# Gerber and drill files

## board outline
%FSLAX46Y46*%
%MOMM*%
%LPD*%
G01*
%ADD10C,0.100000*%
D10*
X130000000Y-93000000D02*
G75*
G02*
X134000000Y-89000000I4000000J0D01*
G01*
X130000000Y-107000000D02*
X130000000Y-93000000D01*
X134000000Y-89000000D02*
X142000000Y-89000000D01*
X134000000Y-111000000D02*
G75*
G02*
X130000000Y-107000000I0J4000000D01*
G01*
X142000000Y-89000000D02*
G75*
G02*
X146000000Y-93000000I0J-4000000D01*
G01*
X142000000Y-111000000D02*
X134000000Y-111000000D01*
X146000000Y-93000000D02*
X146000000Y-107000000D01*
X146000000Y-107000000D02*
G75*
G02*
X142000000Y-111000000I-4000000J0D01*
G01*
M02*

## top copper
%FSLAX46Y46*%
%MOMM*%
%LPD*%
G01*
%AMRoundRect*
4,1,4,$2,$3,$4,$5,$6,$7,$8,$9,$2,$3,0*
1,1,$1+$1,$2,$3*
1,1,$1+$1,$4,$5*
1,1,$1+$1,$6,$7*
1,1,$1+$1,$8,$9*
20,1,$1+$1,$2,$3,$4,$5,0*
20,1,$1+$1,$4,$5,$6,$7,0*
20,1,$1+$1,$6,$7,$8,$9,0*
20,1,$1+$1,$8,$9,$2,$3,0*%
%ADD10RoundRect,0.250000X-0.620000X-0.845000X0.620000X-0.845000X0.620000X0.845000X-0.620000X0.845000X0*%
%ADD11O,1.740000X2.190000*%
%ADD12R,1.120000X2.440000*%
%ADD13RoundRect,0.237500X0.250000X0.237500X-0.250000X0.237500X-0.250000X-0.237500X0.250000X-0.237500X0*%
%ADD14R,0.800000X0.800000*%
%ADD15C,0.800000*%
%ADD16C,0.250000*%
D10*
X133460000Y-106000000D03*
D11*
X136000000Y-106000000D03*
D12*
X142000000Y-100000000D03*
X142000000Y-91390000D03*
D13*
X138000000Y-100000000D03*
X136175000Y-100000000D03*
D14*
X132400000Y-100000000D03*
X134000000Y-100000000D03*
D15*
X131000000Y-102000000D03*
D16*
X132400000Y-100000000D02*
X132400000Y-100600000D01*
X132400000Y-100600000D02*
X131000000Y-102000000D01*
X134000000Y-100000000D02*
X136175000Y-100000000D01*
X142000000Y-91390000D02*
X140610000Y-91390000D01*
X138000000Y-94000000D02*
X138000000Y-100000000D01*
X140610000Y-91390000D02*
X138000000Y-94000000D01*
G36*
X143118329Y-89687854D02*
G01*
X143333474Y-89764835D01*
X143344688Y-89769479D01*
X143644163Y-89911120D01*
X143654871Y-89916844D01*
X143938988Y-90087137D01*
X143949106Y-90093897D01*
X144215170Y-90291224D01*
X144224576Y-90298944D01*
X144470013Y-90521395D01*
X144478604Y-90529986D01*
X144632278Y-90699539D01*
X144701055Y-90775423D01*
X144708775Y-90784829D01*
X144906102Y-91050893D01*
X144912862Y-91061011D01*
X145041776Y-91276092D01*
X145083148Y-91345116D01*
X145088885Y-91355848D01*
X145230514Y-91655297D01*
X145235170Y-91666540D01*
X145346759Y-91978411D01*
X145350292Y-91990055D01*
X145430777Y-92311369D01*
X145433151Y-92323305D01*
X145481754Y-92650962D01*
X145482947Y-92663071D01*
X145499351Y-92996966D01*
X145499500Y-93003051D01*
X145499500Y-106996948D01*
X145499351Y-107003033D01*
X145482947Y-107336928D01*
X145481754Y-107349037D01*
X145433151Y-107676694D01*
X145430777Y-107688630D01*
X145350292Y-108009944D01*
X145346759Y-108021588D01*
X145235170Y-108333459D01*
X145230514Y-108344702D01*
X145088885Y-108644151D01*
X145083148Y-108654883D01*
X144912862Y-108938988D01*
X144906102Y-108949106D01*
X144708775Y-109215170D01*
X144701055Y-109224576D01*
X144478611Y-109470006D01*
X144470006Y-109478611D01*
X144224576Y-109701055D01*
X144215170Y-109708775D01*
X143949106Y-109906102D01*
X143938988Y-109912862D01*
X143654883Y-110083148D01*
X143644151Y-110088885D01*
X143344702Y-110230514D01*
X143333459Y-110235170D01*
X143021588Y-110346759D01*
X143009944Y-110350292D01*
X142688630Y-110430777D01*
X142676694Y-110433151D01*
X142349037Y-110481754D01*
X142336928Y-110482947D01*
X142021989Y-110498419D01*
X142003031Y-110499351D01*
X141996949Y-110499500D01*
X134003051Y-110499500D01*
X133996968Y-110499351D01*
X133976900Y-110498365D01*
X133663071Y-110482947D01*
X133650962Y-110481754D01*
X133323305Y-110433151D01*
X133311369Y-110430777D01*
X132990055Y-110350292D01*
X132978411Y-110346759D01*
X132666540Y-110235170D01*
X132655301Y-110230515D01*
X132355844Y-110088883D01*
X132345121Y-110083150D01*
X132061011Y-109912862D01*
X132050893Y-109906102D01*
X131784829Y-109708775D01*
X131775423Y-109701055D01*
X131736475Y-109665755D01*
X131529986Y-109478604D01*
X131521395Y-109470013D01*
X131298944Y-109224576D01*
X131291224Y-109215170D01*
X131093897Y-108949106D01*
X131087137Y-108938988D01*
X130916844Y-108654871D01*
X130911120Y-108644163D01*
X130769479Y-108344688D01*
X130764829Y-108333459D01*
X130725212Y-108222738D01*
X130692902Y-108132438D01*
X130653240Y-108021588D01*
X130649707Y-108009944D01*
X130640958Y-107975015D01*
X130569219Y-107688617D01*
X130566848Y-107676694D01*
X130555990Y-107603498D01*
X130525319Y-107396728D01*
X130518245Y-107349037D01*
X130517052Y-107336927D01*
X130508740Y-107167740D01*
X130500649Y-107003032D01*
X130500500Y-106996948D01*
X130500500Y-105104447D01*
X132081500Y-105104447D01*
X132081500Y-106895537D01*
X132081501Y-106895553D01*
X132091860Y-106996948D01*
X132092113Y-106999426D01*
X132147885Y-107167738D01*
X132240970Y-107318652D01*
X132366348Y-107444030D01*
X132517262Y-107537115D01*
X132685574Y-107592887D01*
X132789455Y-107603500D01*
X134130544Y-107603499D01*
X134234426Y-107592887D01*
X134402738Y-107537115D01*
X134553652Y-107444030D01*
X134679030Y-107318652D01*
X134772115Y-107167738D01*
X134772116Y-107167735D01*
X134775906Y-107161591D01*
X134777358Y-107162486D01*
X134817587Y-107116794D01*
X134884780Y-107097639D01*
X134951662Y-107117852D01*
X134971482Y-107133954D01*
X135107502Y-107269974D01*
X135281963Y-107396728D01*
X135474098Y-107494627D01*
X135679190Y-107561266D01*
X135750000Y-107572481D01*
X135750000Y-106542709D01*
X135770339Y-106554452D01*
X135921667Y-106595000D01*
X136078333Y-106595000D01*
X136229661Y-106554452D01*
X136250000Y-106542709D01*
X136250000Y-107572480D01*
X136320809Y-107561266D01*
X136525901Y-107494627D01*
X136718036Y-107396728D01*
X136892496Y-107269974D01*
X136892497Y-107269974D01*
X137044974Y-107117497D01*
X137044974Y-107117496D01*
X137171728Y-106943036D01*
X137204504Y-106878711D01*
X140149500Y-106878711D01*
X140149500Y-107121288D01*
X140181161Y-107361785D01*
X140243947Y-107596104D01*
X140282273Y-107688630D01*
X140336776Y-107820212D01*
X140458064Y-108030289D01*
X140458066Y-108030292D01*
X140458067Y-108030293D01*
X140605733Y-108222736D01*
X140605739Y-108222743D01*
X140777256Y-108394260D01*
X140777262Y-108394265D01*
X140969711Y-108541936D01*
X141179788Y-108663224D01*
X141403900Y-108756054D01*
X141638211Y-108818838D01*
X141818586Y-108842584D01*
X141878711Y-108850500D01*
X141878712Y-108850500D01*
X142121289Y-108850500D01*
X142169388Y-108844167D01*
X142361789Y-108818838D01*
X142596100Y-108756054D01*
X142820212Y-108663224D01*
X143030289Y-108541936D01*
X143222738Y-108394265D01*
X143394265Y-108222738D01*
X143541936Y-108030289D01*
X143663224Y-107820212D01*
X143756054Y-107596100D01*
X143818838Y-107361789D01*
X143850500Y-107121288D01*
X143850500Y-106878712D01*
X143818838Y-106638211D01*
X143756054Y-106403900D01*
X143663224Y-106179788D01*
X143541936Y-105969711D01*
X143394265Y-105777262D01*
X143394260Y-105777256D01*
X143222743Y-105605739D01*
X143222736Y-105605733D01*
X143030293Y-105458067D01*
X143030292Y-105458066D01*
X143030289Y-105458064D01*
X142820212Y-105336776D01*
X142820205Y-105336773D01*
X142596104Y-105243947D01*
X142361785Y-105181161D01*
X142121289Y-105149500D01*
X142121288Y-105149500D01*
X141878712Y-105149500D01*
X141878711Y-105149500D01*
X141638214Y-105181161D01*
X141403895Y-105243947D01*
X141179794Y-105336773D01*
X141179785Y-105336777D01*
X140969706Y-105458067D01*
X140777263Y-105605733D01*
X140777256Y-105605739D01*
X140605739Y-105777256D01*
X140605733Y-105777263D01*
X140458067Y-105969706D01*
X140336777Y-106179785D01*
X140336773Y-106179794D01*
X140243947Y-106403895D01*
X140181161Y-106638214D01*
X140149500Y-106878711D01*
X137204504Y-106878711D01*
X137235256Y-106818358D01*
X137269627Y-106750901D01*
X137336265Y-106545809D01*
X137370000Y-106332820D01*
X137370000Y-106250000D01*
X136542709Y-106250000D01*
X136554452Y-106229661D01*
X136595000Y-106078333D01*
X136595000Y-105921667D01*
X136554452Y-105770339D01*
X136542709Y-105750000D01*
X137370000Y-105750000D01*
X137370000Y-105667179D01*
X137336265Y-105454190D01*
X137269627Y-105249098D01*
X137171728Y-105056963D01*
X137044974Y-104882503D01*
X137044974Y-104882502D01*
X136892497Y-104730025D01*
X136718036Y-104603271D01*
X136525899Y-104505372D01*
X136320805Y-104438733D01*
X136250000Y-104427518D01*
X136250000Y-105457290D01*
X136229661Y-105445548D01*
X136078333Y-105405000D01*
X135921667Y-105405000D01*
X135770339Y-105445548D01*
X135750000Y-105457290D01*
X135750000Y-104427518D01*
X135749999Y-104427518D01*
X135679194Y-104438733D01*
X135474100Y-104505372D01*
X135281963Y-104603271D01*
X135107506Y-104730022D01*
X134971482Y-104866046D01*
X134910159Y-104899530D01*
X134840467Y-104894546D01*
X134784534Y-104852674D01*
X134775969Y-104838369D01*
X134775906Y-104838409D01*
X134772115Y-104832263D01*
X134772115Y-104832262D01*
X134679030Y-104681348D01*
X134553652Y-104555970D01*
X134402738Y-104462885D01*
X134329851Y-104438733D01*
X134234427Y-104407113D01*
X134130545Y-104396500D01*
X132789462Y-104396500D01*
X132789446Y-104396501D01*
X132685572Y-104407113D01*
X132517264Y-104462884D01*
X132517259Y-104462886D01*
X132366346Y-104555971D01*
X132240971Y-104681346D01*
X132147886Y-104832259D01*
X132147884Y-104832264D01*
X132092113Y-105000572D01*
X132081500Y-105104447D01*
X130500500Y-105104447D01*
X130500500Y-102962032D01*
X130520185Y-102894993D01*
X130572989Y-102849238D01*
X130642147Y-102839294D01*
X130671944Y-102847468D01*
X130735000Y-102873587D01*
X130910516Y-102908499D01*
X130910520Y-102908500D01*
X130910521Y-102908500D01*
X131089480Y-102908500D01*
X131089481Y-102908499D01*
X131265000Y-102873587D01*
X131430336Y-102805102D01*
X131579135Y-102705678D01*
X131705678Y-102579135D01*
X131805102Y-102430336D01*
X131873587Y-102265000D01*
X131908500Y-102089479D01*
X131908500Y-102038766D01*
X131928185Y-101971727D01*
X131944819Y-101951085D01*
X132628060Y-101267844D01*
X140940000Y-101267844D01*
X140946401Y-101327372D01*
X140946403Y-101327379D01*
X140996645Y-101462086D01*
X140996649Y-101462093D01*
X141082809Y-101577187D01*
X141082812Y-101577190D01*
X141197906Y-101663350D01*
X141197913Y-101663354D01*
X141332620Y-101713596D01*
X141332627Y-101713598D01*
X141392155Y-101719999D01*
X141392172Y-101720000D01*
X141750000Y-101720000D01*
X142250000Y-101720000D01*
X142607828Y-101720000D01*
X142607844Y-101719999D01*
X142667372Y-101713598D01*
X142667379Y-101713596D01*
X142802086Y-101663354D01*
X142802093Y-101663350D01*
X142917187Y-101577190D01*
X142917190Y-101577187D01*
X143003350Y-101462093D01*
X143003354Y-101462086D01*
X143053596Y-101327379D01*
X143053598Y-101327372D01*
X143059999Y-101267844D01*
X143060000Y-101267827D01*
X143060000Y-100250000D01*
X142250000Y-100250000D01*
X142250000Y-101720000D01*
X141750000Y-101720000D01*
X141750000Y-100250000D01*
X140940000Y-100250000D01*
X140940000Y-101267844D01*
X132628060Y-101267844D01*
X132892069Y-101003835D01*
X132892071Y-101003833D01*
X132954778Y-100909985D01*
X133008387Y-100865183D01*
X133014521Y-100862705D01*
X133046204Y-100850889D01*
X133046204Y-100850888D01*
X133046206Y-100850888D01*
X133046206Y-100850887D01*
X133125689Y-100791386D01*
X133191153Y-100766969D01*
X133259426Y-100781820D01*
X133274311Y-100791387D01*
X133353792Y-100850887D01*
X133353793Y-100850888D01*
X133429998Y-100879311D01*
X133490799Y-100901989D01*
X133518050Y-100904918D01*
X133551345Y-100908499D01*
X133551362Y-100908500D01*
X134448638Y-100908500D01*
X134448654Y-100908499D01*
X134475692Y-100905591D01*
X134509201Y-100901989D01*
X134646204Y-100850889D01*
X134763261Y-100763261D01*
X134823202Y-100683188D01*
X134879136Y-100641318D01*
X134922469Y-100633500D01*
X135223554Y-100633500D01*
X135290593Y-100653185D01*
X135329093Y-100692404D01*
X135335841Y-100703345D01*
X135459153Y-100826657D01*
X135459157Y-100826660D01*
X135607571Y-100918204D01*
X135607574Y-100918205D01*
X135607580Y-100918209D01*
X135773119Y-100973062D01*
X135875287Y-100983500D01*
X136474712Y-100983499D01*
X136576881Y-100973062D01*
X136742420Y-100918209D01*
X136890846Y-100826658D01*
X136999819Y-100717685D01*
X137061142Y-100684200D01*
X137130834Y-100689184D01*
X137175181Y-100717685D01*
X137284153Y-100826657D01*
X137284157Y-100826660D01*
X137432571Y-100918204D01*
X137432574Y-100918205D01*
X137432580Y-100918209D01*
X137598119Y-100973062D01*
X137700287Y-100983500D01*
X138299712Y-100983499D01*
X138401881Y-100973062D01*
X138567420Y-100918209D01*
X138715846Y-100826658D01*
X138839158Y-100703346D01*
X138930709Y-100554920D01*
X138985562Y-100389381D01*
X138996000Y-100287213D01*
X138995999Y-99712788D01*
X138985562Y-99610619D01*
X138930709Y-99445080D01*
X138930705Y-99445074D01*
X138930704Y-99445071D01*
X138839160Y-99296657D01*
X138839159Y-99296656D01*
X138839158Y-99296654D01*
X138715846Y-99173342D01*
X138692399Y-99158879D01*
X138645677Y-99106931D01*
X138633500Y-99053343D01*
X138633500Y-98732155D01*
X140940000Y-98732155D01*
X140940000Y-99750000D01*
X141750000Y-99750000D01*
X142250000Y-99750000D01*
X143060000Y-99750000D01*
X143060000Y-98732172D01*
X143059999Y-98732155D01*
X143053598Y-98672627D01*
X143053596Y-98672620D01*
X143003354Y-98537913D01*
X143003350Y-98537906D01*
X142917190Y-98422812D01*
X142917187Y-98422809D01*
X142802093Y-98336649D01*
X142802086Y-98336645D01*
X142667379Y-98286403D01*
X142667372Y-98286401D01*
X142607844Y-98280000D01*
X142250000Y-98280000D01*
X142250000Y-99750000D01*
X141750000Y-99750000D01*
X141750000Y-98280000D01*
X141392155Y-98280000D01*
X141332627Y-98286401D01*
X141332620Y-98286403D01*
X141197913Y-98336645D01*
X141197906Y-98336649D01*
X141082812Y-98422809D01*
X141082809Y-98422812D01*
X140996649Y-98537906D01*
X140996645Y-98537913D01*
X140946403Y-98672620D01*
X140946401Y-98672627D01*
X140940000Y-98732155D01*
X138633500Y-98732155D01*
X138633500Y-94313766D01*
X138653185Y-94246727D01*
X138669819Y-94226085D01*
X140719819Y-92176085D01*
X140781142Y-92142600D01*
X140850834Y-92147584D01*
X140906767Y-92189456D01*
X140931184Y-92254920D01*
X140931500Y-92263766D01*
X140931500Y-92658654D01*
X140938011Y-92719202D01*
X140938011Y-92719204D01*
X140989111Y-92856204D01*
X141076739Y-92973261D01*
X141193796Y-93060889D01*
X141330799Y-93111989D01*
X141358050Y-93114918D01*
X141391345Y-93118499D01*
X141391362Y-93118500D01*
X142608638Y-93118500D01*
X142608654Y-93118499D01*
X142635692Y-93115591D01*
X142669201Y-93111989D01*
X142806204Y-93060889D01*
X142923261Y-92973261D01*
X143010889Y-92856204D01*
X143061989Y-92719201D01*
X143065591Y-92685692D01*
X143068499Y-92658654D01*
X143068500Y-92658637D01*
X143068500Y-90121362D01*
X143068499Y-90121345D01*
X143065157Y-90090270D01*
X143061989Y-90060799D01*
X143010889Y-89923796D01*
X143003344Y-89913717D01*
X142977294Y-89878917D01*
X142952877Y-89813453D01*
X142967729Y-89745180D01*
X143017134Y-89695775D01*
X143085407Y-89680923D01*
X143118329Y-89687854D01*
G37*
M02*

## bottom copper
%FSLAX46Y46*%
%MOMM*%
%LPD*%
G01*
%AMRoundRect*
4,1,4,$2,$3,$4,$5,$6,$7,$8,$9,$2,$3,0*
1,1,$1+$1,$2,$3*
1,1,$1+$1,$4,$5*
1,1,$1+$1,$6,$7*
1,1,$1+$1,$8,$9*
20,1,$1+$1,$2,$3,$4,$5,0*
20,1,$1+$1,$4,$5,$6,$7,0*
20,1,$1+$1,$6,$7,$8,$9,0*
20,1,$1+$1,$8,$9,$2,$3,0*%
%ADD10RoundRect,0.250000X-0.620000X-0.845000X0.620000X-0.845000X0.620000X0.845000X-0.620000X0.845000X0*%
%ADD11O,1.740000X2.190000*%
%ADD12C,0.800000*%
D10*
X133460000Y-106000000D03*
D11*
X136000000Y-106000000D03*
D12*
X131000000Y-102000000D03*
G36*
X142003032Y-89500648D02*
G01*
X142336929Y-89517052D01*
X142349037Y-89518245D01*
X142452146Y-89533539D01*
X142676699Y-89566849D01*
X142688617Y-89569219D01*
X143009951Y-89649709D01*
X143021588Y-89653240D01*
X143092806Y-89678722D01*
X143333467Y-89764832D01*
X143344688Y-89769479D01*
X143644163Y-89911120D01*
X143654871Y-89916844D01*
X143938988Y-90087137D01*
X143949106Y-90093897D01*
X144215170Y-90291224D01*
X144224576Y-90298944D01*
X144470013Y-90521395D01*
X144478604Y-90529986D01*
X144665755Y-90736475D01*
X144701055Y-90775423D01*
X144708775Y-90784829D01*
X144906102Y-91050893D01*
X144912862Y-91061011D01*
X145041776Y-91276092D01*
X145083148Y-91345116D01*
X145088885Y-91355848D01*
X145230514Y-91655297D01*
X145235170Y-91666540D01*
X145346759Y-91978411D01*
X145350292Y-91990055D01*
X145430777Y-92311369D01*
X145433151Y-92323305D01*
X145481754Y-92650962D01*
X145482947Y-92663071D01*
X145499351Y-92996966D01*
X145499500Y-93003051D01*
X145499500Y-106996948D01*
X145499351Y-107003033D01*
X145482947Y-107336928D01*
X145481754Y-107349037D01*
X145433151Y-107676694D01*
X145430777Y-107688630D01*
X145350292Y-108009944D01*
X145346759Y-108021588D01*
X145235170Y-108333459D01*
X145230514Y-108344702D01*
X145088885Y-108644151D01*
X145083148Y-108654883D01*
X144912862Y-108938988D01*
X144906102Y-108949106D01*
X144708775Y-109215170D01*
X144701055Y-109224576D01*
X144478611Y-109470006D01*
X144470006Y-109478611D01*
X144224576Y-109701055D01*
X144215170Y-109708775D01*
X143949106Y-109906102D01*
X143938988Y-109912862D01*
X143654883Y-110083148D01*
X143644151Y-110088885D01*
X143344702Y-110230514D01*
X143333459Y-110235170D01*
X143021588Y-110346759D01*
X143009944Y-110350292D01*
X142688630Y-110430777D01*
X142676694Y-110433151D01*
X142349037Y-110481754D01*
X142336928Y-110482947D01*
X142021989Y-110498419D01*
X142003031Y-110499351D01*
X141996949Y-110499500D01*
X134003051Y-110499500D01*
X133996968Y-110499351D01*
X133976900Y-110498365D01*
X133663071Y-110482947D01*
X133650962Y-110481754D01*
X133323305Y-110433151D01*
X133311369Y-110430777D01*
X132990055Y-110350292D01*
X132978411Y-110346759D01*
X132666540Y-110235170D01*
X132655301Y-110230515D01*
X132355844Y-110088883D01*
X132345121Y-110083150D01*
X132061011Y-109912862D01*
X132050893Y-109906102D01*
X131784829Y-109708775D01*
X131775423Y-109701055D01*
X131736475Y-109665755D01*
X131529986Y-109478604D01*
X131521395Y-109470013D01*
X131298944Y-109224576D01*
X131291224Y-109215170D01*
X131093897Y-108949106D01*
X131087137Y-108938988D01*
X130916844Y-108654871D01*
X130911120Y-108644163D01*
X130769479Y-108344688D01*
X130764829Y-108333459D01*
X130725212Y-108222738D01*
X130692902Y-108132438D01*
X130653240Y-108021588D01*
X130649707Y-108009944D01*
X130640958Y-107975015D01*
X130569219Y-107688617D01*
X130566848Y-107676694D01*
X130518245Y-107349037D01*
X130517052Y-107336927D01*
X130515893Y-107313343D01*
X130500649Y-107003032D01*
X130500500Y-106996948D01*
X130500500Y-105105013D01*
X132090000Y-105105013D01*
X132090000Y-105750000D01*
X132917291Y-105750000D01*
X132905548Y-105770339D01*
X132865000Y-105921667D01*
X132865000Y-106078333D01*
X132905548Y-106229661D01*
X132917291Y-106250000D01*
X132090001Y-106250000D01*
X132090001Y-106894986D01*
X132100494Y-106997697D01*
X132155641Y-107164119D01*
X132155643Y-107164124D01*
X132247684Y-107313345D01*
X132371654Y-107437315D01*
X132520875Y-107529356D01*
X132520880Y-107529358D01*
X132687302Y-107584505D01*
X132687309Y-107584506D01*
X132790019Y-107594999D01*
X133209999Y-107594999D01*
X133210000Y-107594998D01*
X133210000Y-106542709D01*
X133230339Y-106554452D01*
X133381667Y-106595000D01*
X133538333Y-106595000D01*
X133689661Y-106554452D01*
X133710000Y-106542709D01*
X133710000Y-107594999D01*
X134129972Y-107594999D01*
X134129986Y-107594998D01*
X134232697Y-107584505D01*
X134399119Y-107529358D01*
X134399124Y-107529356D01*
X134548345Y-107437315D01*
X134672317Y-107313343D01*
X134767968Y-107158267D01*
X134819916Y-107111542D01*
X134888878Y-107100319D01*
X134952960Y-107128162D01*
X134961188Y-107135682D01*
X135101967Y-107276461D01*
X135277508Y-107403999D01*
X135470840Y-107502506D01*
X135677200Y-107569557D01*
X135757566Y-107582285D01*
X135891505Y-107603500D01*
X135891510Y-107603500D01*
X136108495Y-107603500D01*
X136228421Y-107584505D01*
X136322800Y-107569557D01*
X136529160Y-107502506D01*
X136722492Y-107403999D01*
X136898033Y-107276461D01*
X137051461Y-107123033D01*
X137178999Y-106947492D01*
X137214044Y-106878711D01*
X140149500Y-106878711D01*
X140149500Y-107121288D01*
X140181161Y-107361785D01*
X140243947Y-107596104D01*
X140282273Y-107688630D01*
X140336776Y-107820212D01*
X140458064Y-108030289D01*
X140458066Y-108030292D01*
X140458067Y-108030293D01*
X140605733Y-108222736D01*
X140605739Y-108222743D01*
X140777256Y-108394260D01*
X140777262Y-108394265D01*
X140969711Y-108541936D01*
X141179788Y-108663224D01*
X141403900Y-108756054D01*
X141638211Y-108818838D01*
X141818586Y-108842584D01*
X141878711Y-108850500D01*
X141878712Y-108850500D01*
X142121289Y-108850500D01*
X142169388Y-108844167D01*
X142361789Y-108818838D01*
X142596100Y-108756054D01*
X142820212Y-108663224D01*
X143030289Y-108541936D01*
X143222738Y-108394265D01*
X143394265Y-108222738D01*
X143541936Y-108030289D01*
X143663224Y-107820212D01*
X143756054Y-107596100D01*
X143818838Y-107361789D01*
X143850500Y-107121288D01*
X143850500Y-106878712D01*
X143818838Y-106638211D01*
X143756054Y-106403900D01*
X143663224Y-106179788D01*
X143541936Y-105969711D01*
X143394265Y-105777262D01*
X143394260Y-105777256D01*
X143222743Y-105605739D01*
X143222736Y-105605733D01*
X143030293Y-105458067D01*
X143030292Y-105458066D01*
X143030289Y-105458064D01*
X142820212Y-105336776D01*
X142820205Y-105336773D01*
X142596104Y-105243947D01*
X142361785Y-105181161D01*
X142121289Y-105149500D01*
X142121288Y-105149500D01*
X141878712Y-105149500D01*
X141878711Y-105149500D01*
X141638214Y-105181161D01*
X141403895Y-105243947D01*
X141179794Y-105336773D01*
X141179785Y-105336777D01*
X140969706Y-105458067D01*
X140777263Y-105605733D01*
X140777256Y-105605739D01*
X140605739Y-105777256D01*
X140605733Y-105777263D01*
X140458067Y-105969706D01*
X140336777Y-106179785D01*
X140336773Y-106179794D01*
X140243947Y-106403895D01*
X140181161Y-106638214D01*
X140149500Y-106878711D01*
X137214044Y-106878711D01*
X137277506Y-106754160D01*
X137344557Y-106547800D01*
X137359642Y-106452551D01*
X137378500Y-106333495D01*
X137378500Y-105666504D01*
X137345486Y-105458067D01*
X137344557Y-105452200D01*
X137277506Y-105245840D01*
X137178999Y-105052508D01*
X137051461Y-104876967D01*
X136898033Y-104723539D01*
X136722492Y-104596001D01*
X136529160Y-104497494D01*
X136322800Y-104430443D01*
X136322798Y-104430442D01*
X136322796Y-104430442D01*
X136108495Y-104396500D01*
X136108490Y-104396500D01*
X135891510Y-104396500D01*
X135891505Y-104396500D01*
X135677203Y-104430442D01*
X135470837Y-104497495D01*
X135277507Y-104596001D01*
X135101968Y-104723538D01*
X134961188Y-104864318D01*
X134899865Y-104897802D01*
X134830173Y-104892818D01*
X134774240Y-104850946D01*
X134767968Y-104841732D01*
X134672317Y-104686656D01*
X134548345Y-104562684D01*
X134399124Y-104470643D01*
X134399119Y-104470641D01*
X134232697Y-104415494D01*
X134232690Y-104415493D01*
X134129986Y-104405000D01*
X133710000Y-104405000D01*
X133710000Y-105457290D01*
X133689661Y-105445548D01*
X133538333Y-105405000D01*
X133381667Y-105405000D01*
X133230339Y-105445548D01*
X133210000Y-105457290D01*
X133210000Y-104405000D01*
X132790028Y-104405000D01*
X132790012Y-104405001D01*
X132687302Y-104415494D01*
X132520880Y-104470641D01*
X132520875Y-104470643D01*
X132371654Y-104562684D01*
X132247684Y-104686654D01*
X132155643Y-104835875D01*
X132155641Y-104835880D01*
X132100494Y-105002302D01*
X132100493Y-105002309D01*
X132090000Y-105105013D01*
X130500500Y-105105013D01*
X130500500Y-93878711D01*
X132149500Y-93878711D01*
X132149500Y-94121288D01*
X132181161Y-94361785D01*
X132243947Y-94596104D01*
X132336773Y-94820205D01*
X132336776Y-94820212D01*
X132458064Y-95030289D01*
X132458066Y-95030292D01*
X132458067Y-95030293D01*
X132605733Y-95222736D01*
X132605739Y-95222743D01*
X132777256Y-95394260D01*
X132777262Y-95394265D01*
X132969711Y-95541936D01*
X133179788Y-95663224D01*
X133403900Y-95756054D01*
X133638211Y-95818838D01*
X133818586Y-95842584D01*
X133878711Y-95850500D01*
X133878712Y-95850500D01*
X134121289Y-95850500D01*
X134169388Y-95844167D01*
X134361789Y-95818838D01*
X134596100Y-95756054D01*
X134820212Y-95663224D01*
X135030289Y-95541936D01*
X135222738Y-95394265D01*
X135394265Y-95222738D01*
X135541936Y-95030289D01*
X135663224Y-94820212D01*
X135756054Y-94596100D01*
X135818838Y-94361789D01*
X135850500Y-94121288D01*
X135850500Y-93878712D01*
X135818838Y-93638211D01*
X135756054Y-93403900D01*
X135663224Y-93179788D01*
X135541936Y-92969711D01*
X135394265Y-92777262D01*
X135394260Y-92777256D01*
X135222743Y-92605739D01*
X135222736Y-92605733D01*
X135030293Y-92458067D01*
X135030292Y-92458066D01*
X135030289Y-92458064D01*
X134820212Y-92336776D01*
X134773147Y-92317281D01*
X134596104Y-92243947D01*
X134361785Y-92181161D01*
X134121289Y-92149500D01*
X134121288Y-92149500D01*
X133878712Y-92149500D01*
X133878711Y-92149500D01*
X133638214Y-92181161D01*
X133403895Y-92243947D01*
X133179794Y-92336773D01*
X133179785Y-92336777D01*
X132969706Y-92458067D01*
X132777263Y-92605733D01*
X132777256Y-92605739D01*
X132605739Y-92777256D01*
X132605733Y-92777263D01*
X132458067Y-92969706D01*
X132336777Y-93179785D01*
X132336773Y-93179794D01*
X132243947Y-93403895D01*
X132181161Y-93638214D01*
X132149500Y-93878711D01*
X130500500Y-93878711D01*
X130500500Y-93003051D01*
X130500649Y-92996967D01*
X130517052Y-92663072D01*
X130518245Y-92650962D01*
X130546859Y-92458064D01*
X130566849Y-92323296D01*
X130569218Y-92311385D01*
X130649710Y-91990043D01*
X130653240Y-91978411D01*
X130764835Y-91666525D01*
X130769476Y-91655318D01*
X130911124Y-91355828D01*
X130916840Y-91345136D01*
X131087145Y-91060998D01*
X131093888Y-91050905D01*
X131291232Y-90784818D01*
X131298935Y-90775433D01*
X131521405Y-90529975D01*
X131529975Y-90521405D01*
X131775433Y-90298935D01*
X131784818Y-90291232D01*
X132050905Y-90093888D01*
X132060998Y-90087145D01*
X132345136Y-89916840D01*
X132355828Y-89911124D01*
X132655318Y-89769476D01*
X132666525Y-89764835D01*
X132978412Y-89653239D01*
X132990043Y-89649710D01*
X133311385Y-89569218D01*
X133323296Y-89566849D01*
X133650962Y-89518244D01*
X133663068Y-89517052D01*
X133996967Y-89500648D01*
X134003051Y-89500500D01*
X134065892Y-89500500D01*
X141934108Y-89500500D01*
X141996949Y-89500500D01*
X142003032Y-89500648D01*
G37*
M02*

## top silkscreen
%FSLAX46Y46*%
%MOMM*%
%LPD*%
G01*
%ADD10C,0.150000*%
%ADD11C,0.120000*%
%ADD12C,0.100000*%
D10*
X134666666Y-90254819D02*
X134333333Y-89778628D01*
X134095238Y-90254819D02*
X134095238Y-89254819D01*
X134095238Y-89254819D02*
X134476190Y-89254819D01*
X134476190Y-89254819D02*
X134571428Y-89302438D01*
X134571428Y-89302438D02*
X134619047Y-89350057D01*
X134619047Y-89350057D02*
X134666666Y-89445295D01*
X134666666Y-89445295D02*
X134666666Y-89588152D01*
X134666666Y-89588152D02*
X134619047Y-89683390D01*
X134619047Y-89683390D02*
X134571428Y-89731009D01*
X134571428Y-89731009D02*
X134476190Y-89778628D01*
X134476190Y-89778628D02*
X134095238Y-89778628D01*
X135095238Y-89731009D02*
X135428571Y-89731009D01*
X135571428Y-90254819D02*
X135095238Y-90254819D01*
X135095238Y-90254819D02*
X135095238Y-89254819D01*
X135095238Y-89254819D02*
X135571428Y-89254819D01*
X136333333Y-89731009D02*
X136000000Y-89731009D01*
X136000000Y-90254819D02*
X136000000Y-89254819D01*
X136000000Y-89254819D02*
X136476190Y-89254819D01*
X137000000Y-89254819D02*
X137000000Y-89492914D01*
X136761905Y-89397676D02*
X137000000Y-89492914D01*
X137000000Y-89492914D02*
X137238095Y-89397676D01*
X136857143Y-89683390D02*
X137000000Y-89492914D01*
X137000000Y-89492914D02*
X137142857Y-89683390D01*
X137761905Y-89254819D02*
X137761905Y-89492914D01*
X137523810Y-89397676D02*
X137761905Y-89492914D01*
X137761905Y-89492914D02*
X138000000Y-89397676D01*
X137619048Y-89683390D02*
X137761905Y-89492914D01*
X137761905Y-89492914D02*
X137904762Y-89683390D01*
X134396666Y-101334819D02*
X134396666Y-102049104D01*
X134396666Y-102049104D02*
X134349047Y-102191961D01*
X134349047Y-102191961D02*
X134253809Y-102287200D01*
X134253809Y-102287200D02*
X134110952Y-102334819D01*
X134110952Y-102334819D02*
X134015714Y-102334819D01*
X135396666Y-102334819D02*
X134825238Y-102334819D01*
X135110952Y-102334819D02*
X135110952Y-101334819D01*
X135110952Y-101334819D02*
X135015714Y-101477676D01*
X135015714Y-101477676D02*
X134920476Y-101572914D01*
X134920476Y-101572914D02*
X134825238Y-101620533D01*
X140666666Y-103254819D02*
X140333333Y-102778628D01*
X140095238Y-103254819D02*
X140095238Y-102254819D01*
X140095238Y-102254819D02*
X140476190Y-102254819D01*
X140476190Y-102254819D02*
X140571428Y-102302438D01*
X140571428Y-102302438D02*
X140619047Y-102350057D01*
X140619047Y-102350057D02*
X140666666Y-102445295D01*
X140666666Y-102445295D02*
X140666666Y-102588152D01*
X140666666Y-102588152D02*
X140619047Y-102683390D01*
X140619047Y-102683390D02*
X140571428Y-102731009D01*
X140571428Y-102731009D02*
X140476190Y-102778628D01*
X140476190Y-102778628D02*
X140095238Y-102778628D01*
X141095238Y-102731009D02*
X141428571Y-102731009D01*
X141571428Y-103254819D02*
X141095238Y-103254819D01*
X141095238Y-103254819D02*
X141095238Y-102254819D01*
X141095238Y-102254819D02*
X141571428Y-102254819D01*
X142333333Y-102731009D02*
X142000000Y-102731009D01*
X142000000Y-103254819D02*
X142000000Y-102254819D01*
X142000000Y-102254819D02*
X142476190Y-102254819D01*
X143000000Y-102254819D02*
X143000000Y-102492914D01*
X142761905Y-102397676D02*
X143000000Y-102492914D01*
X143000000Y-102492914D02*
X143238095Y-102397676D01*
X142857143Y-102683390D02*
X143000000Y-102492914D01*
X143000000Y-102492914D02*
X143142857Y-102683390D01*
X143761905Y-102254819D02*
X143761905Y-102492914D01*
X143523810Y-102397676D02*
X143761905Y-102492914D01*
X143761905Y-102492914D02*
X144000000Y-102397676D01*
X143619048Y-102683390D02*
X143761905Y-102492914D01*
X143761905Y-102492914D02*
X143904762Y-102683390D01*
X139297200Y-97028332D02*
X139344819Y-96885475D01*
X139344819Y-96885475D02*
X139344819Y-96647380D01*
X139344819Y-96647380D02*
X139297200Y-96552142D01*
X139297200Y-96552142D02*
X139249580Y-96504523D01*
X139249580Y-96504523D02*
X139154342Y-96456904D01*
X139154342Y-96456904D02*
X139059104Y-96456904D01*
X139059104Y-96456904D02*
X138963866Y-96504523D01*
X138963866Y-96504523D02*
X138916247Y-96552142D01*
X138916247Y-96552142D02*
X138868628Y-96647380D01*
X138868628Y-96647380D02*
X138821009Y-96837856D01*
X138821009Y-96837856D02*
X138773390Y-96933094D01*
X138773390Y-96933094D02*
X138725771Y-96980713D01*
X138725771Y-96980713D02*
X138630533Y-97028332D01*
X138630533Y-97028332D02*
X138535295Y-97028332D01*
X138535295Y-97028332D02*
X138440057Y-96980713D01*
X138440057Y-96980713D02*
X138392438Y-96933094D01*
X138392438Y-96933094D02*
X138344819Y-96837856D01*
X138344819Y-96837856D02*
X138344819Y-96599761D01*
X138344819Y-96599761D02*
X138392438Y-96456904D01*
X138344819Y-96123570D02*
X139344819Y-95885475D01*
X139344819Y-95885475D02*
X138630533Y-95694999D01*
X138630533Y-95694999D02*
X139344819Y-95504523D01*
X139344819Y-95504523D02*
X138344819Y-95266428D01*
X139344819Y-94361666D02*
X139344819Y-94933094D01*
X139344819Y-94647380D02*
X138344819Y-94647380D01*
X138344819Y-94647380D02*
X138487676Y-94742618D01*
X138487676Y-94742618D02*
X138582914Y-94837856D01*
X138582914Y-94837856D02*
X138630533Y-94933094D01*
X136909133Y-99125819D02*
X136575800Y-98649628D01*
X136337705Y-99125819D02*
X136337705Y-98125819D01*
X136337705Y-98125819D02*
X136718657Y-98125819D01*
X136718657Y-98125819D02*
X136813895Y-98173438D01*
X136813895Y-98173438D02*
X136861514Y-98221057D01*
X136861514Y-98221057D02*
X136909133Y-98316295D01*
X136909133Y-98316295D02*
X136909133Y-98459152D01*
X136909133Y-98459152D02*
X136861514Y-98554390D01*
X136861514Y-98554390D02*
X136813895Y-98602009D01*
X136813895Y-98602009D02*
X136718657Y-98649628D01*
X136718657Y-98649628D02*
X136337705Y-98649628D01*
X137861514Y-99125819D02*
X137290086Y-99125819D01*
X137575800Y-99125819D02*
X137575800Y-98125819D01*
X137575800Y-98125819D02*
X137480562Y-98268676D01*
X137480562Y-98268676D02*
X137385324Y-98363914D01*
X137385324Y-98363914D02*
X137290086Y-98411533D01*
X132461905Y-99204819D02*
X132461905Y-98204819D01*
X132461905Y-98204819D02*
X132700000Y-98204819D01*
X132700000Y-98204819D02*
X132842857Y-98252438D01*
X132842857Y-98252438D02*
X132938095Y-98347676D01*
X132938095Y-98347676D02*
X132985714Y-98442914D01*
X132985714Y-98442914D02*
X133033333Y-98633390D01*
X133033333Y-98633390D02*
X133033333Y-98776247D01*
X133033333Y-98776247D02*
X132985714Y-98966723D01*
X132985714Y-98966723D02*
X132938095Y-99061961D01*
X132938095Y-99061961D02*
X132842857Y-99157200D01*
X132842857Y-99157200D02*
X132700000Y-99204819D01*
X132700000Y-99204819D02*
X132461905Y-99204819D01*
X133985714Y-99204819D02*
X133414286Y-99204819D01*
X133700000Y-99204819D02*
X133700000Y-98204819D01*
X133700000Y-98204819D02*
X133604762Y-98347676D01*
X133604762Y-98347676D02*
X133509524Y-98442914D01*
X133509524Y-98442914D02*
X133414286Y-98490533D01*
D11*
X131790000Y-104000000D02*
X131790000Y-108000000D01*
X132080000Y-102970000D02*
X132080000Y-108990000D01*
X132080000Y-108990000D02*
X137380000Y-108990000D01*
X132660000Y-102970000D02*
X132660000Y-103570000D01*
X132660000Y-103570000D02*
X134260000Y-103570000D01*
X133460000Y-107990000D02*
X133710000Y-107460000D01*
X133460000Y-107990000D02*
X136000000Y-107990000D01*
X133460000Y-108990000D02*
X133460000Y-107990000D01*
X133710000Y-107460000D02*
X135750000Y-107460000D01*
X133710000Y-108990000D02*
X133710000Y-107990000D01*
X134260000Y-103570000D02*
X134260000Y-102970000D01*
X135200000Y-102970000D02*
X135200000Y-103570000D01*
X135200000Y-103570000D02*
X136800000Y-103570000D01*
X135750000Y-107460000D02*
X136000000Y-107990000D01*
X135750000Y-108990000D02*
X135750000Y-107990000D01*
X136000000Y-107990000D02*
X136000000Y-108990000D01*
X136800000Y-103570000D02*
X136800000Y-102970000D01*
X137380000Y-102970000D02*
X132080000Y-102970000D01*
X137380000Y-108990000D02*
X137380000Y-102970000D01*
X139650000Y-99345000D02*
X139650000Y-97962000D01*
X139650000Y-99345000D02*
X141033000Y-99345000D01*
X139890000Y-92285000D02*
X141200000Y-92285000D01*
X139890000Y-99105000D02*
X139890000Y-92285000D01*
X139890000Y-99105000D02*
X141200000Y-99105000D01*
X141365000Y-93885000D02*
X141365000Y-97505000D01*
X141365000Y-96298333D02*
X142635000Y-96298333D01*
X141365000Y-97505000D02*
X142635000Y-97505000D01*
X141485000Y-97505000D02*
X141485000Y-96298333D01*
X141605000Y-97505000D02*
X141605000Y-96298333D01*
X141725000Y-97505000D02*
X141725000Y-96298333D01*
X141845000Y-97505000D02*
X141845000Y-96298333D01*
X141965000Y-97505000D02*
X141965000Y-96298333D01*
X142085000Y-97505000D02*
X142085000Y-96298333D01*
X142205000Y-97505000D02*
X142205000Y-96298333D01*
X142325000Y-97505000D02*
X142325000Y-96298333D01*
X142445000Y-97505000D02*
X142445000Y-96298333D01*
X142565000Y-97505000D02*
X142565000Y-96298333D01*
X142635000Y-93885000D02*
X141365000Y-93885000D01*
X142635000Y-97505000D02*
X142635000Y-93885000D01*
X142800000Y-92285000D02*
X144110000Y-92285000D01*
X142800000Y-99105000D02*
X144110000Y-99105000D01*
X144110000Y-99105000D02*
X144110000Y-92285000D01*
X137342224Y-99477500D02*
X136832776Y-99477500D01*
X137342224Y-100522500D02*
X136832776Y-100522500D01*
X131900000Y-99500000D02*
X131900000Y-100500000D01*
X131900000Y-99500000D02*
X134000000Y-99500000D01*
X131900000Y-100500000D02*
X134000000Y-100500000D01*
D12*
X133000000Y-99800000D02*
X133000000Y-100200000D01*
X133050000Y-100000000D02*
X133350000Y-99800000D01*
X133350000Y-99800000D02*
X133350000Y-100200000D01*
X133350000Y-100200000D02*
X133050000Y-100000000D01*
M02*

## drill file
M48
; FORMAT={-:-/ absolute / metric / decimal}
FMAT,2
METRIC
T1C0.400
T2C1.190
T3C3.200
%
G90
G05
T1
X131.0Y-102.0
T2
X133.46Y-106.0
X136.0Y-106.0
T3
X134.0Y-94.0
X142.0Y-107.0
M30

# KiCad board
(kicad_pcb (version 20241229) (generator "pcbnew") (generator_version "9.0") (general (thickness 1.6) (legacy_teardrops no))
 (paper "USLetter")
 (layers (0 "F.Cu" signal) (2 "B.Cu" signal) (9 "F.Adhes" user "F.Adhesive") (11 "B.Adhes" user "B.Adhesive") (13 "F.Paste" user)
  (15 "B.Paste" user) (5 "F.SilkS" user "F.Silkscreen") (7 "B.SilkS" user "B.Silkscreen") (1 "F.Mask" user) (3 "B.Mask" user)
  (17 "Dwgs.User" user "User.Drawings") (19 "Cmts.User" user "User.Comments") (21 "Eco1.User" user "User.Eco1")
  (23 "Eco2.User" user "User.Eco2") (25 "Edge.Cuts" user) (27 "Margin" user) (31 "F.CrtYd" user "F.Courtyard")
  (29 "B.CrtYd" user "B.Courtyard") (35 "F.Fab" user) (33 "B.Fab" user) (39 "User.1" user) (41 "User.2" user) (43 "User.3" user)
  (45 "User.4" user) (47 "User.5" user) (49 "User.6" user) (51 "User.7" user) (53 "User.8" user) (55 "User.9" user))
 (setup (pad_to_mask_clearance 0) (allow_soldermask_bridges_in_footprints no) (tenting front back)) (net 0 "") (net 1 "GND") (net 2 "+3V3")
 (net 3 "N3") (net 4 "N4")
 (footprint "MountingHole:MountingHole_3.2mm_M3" (layer "F.Cu") (at 134 94)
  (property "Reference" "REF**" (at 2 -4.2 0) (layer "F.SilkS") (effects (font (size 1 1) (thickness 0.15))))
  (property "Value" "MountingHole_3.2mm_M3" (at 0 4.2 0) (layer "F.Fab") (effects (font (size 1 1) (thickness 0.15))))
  (pad "" np_thru_hole circle (at 0 0) (size 3.2 3.2) (drill 3.2) (layers "*.Cu" "*.Mask")))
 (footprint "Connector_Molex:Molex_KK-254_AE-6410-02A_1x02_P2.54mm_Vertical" (layer "F.Cu") (at 133.46 106)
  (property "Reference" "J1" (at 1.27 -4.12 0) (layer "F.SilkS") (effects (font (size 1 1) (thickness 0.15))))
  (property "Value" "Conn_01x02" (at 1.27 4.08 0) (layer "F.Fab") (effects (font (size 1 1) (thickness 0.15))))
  (fp_line (start -1.67 -2) (end -1.67 2) (stroke (width 0.12) (type solid)) (layer "F.SilkS"))
  (fp_line (start -1.38 -3.03) (end -1.38 2.99) (stroke (width 0.12) (type solid)) (layer "F.SilkS"))
  (fp_line (start -1.38 2.99) (end 3.92 2.99) (stroke (width 0.12) (type solid)) (layer "F.SilkS"))
  (fp_line (start -0.8 -3.03) (end -0.8 -2.43) (stroke (width 0.12) (type solid)) (layer "F.SilkS"))
  (fp_line (start -0.8 -2.43) (end 0.8 -2.43) (stroke (width 0.12) (type solid)) (layer "F.SilkS"))
  (fp_line (start 0 1.99) (end 0.25 1.46) (stroke (width 0.12) (type solid)) (layer "F.SilkS"))
  (fp_line (start 0 1.99) (end 2.54 1.99) (stroke (width 0.12) (type solid)) (layer "F.SilkS"))
  (fp_line (start 0 2.99) (end 0 1.99) (stroke (width 0.12) (type solid)) (layer "F.SilkS"))
  (fp_line (start 0.25 1.46) (end 2.29 1.46) (stroke (width 0.12) (type solid)) (layer "F.SilkS"))
  (fp_line (start 0.25 2.99) (end 0.25 1.99) (stroke (width 0.12) (type solid)) (layer "F.SilkS"))
  (fp_line (start 0.8 -2.43) (end 0.8 -3.03) (stroke (width 0.12) (type solid)) (layer "F.SilkS"))
  (fp_line (start 1.74 -3.03) (end 1.74 -2.43) (stroke (width 0.12) (type solid)) (layer "F.SilkS"))
  (fp_line (start 1.74 -2.43) (end 3.34 -2.43) (stroke (width 0.12) (type solid)) (layer "F.SilkS"))
  (fp_line (start 2.29 1.46) (end 2.54 1.99) (stroke (width 0.12) (type solid)) (layer "F.SilkS"))
  (fp_line (start 2.29 2.99) (end 2.29 1.99) (stroke (width 0.12) (type solid)) (layer "F.SilkS"))
  (fp_line (start 2.54 1.99) (end 2.54 2.99) (stroke (width 0.12) (type solid)) (layer "F.SilkS"))
  (fp_line (start 3.34 -2.43) (end 3.34 -3.03) (stroke (width 0.12) (type solid)) (layer "F.SilkS"))
  (fp_line (start 3.92 -3.03) (end -1.38 -3.03) (stroke (width 0.12) (type solid)) (layer "F.SilkS"))
  (fp_line (start 3.92 2.99) (end 3.92 -3.03) (stroke (width 0.12) (type solid)) (layer "F.SilkS"))
  (pad "1" thru_hole roundrect (at 0 0) (size 1.74 2.19) (drill 1.19) (layers "*.Cu" "*.Mask") (remove_unused_layers no)
   (roundrect_rratio 0.143678) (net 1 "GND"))
  (pad "2" thru_hole oval (at 2.54 0) (size 1.74 2.19) (drill 1.19) (layers "*.Cu" "*.Mask") (remove_unused_layers no) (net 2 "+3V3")))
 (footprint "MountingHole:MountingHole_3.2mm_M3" (layer "F.Cu") (at 142 107)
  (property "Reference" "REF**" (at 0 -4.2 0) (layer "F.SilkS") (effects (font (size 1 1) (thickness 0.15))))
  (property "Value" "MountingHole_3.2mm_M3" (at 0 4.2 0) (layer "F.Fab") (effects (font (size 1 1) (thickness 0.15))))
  (pad "" np_thru_hole circle (at 0 0) (size 3.2 3.2) (drill 3.2) (layers "*.Cu" "*.Mask")))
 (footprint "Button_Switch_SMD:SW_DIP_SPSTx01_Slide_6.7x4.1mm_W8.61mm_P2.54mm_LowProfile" (layer "F.Cu") (at 142 95.695 90)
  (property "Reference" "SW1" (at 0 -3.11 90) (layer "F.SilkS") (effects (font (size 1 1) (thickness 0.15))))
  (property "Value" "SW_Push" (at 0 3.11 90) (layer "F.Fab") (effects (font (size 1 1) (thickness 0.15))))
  (fp_line (start -3.65 -2.35) (end -2.267 -2.35) (stroke (width 0.12) (type solid)) (layer "F.SilkS"))
  (fp_line (start -3.65 -2.35) (end -3.65 -0.967) (stroke (width 0.12) (type solid)) (layer "F.SilkS"))
  (fp_line (start 3.41 -2.11) (end 3.41 -0.8) (stroke (width 0.12) (type solid)) (layer "F.SilkS"))
  (fp_line (start -3.41 -2.11) (end 3.41 -2.11) (stroke (width 0.12) (type solid)) (layer "F.SilkS"))
  (fp_line (start -3.41 -2.11) (end -3.41 -0.8) (stroke (width 0.12) (type solid)) (layer "F.SilkS"))
  (fp_line (start 1.81 -0.635) (end -1.81 -0.635) (stroke (width 0.12) (type solid)) (layer "F.SilkS"))
  (fp_line (start -0.603333 -0.635) (end -0.603333 0.635) (stroke (width 0.12) (type solid)) (layer "F.SilkS"))
  (fp_line (start -1.81 -0.635) (end -1.81 0.635) (stroke (width 0.12) (type solid)) (layer "F.SilkS"))
  (fp_line (start -1.81 -0.515) (end -0.603333 -0.515) (stroke (width 0.12) (type solid)) (layer "F.SilkS"))
  (fp_line (start -1.81 -0.395) (end -0.603333 -0.395) (stroke (width 0.12) (type solid)) (layer "F.SilkS"))
  (fp_line (start -1.81 -0.275) (end -0.603333 -0.275) (stroke (width 0.12) (type solid)) (layer "F.SilkS"))
  (fp_line (start -1.81 -0.155) (end -0.603333 -0.155) (stroke (width 0.12) (type solid)) (layer "F.SilkS"))
  (fp_line (start -1.81 -0.035) (end -0.603333 -0.035) (stroke (width 0.12) (type solid)) (layer "F.SilkS"))
  (fp_line (start -1.81 0.085) (end -0.603333 0.085) (stroke (width 0.12) (type solid)) (layer "F.SilkS"))
  (fp_line (start -1.81 0.205) (end -0.603333 0.205) (stroke (width 0.12) (type solid)) (layer "F.SilkS"))
  (fp_line (start -1.81 0.325) (end -0.603333 0.325) (stroke (width 0.12) (type solid)) (layer "F.SilkS"))
  (fp_line (start -1.81 0.445) (end -0.603333 0.445) (stroke (width 0.12) (type solid)) (layer "F.SilkS"))
  (fp_line (start -1.81 0.565) (end -0.603333 0.565) (stroke (width 0.12) (type solid)) (layer "F.SilkS"))
  (fp_line (start 1.81 0.635) (end 1.81 -0.635) (stroke (width 0.12) (type solid)) (layer "F.SilkS"))
  (fp_line (start -1.81 0.635) (end 1.81 0.635) (stroke (width 0.12) (type solid)) (layer "F.SilkS"))
  (fp_line (start 3.41 0.8) (end 3.41 2.11) (stroke (width 0.12) (type solid)) (layer "F.SilkS"))
  (fp_line (start -3.41 0.8) (end -3.41 2.11) (stroke (width 0.12) (type solid)) (layer "F.SilkS"))
  (fp_line (start -3.41 2.11) (end 3.41 2.11) (stroke (width 0.12) (type solid)) (layer "F.SilkS"))
  (pad "1" smd rect (at -4.305 0 90) (size 2.44 1.12) (layers "F.Cu" "F.Mask" "F.Paste") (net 2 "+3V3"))
  (pad "2" smd rect (at 4.305 0 90) (size 2.44 1.12) (layers "F.Cu" "F.Mask" "F.Paste") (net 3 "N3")))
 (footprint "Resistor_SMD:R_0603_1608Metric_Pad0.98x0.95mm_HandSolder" (layer "F.Cu") (at 137.0875 100 180)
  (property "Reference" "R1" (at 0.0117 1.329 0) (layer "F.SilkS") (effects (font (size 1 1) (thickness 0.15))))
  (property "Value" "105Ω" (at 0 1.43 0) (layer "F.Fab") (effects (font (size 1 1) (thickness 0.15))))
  (fp_line (start -0.254724 0.5225) (end 0.254724 0.5225) (stroke (width 0.12) (type solid)) (layer "F.SilkS"))
  (fp_line (start -0.254724 -0.5225) (end 0.254724 -0.5225) (stroke (width 0.12) (type solid)) (layer "F.SilkS"))
  (pad "1" smd roundrect (at -0.9125 0 180) (size 0.975 0.95) (layers "F.Cu" "F.Mask" "F.Paste") (roundrect_rratio 0.25) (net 3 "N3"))
  (pad "2" smd roundrect (at 0.9125 0 180) (size 0.975 0.95) (layers "F.Cu" "F.Mask" "F.Paste") (roundrect_rratio 0.25) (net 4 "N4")))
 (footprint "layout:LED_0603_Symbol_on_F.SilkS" (layer "F.Cu") (at 133.2 100)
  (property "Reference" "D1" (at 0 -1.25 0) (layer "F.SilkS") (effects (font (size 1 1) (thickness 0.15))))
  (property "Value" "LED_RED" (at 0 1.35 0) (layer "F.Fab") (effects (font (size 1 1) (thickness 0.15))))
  (fp_line (start -1.3 -0.5) (end -1.3 0.5) (stroke (width 0.12) (type solid)) (layer "F.SilkS"))
  (fp_line (start -1.3 -0.5) (end 0.8 -0.5) (stroke (width 0.12) (type solid)) (layer "F.SilkS"))
  (fp_line (start -1.3 0.5) (end 0.8 0.5) (stroke (width 0.12) (type solid)) (layer "F.SilkS"))
  (fp_line (start -0.2 -0.2) (end -0.2 0.2) (stroke (width 0.1) (type solid)) (layer "F.SilkS"))
  (fp_line (start -0.15 0) (end 0.15 -0.2) (stroke (width 0.1) (type solid)) (layer "F.SilkS"))
  (fp_line (start 0.15 -0.2) (end 0.15 0.2) (stroke (width 0.1) (type solid)) (layer "F.SilkS"))
  (fp_line (start 0.15 0.2) (end -0.15 0) (stroke (width 0.1) (type solid)) (layer "F.SilkS"))
  (pad "1" smd rect (at -0.8 0 180) (size 0.8 0.8) (layers "F.Cu" "F.Mask" "F.Paste") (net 1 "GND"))
  (pad "2" smd rect (at 0.8 0 180) (size 0.8 0.8) (layers "F.Cu" "F.Mask" "F.Paste") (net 4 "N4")))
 (gr_arc (start 130 93) (mid 131.171573 90.171573) (end 134 89) (stroke (width 0.1) (type default)) (layer "Edge.Cuts"))
 (gr_line (start 130 107) (end 130 93) (stroke (width 0.1) (type default)) (layer "Edge.Cuts"))
 (gr_line (start 134 89) (end 142 89) (stroke (width 0.1) (type default)) (layer "Edge.Cuts"))
 (gr_arc (start 134 111) (mid 131.171573 109.828427) (end 130 107) (stroke (width 0.1) (type default)) (layer "Edge.Cuts"))
 (gr_arc (start 142 89) (mid 144.828427 90.171573) (end 146 93) (stroke (width 0.1) (type default)) (layer "Edge.Cuts"))
 (gr_line (start 142 111) (end 134 111) (stroke (width 0.1) (type default)) (layer "Edge.Cuts"))
 (gr_line (start 146 93) (end 146 107) (stroke (width 0.1) (type default)) (layer "Edge.Cuts"))
 (gr_arc (start 146 107) (mid 144.828427 109.828427) (end 142 111) (stroke (width 0.1) (type default)) (layer "Edge.Cuts"))
 (segment (start 132.4 100) (end 132.4 100.6) (width 0.25) (layer "F.Cu") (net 1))
 (segment (start 132.4 100.6) (end 131 102) (width 0.25) (layer "F.Cu") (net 1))
 (via (at 131 102) (size 0.8) (drill 0.4) (layers "F.Cu" "B.Cu") (free yes) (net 1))
 (segment (start 134 100) (end 136.175 100) (width 0.25) (layer "F.Cu") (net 4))
 (segment (start 142 91.39) (end 140.61 91.39) (width 0.25) (layer "F.Cu") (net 3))
 (segment (start 138 94) (end 138 100) (width 0.25) (layer "F.Cu") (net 3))
 (segment (start 140.61 91.39) (end 138 94) (width 0.25) (layer "F.Cu") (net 3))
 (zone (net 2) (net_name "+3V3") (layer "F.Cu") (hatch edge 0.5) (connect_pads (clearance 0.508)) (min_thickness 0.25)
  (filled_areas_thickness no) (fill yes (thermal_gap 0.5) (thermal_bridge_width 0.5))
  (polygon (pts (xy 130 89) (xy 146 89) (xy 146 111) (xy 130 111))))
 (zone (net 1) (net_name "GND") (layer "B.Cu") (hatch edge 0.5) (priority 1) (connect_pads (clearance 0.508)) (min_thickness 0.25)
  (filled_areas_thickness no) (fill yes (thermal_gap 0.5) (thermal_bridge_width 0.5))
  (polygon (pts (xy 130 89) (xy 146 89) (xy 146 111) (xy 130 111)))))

